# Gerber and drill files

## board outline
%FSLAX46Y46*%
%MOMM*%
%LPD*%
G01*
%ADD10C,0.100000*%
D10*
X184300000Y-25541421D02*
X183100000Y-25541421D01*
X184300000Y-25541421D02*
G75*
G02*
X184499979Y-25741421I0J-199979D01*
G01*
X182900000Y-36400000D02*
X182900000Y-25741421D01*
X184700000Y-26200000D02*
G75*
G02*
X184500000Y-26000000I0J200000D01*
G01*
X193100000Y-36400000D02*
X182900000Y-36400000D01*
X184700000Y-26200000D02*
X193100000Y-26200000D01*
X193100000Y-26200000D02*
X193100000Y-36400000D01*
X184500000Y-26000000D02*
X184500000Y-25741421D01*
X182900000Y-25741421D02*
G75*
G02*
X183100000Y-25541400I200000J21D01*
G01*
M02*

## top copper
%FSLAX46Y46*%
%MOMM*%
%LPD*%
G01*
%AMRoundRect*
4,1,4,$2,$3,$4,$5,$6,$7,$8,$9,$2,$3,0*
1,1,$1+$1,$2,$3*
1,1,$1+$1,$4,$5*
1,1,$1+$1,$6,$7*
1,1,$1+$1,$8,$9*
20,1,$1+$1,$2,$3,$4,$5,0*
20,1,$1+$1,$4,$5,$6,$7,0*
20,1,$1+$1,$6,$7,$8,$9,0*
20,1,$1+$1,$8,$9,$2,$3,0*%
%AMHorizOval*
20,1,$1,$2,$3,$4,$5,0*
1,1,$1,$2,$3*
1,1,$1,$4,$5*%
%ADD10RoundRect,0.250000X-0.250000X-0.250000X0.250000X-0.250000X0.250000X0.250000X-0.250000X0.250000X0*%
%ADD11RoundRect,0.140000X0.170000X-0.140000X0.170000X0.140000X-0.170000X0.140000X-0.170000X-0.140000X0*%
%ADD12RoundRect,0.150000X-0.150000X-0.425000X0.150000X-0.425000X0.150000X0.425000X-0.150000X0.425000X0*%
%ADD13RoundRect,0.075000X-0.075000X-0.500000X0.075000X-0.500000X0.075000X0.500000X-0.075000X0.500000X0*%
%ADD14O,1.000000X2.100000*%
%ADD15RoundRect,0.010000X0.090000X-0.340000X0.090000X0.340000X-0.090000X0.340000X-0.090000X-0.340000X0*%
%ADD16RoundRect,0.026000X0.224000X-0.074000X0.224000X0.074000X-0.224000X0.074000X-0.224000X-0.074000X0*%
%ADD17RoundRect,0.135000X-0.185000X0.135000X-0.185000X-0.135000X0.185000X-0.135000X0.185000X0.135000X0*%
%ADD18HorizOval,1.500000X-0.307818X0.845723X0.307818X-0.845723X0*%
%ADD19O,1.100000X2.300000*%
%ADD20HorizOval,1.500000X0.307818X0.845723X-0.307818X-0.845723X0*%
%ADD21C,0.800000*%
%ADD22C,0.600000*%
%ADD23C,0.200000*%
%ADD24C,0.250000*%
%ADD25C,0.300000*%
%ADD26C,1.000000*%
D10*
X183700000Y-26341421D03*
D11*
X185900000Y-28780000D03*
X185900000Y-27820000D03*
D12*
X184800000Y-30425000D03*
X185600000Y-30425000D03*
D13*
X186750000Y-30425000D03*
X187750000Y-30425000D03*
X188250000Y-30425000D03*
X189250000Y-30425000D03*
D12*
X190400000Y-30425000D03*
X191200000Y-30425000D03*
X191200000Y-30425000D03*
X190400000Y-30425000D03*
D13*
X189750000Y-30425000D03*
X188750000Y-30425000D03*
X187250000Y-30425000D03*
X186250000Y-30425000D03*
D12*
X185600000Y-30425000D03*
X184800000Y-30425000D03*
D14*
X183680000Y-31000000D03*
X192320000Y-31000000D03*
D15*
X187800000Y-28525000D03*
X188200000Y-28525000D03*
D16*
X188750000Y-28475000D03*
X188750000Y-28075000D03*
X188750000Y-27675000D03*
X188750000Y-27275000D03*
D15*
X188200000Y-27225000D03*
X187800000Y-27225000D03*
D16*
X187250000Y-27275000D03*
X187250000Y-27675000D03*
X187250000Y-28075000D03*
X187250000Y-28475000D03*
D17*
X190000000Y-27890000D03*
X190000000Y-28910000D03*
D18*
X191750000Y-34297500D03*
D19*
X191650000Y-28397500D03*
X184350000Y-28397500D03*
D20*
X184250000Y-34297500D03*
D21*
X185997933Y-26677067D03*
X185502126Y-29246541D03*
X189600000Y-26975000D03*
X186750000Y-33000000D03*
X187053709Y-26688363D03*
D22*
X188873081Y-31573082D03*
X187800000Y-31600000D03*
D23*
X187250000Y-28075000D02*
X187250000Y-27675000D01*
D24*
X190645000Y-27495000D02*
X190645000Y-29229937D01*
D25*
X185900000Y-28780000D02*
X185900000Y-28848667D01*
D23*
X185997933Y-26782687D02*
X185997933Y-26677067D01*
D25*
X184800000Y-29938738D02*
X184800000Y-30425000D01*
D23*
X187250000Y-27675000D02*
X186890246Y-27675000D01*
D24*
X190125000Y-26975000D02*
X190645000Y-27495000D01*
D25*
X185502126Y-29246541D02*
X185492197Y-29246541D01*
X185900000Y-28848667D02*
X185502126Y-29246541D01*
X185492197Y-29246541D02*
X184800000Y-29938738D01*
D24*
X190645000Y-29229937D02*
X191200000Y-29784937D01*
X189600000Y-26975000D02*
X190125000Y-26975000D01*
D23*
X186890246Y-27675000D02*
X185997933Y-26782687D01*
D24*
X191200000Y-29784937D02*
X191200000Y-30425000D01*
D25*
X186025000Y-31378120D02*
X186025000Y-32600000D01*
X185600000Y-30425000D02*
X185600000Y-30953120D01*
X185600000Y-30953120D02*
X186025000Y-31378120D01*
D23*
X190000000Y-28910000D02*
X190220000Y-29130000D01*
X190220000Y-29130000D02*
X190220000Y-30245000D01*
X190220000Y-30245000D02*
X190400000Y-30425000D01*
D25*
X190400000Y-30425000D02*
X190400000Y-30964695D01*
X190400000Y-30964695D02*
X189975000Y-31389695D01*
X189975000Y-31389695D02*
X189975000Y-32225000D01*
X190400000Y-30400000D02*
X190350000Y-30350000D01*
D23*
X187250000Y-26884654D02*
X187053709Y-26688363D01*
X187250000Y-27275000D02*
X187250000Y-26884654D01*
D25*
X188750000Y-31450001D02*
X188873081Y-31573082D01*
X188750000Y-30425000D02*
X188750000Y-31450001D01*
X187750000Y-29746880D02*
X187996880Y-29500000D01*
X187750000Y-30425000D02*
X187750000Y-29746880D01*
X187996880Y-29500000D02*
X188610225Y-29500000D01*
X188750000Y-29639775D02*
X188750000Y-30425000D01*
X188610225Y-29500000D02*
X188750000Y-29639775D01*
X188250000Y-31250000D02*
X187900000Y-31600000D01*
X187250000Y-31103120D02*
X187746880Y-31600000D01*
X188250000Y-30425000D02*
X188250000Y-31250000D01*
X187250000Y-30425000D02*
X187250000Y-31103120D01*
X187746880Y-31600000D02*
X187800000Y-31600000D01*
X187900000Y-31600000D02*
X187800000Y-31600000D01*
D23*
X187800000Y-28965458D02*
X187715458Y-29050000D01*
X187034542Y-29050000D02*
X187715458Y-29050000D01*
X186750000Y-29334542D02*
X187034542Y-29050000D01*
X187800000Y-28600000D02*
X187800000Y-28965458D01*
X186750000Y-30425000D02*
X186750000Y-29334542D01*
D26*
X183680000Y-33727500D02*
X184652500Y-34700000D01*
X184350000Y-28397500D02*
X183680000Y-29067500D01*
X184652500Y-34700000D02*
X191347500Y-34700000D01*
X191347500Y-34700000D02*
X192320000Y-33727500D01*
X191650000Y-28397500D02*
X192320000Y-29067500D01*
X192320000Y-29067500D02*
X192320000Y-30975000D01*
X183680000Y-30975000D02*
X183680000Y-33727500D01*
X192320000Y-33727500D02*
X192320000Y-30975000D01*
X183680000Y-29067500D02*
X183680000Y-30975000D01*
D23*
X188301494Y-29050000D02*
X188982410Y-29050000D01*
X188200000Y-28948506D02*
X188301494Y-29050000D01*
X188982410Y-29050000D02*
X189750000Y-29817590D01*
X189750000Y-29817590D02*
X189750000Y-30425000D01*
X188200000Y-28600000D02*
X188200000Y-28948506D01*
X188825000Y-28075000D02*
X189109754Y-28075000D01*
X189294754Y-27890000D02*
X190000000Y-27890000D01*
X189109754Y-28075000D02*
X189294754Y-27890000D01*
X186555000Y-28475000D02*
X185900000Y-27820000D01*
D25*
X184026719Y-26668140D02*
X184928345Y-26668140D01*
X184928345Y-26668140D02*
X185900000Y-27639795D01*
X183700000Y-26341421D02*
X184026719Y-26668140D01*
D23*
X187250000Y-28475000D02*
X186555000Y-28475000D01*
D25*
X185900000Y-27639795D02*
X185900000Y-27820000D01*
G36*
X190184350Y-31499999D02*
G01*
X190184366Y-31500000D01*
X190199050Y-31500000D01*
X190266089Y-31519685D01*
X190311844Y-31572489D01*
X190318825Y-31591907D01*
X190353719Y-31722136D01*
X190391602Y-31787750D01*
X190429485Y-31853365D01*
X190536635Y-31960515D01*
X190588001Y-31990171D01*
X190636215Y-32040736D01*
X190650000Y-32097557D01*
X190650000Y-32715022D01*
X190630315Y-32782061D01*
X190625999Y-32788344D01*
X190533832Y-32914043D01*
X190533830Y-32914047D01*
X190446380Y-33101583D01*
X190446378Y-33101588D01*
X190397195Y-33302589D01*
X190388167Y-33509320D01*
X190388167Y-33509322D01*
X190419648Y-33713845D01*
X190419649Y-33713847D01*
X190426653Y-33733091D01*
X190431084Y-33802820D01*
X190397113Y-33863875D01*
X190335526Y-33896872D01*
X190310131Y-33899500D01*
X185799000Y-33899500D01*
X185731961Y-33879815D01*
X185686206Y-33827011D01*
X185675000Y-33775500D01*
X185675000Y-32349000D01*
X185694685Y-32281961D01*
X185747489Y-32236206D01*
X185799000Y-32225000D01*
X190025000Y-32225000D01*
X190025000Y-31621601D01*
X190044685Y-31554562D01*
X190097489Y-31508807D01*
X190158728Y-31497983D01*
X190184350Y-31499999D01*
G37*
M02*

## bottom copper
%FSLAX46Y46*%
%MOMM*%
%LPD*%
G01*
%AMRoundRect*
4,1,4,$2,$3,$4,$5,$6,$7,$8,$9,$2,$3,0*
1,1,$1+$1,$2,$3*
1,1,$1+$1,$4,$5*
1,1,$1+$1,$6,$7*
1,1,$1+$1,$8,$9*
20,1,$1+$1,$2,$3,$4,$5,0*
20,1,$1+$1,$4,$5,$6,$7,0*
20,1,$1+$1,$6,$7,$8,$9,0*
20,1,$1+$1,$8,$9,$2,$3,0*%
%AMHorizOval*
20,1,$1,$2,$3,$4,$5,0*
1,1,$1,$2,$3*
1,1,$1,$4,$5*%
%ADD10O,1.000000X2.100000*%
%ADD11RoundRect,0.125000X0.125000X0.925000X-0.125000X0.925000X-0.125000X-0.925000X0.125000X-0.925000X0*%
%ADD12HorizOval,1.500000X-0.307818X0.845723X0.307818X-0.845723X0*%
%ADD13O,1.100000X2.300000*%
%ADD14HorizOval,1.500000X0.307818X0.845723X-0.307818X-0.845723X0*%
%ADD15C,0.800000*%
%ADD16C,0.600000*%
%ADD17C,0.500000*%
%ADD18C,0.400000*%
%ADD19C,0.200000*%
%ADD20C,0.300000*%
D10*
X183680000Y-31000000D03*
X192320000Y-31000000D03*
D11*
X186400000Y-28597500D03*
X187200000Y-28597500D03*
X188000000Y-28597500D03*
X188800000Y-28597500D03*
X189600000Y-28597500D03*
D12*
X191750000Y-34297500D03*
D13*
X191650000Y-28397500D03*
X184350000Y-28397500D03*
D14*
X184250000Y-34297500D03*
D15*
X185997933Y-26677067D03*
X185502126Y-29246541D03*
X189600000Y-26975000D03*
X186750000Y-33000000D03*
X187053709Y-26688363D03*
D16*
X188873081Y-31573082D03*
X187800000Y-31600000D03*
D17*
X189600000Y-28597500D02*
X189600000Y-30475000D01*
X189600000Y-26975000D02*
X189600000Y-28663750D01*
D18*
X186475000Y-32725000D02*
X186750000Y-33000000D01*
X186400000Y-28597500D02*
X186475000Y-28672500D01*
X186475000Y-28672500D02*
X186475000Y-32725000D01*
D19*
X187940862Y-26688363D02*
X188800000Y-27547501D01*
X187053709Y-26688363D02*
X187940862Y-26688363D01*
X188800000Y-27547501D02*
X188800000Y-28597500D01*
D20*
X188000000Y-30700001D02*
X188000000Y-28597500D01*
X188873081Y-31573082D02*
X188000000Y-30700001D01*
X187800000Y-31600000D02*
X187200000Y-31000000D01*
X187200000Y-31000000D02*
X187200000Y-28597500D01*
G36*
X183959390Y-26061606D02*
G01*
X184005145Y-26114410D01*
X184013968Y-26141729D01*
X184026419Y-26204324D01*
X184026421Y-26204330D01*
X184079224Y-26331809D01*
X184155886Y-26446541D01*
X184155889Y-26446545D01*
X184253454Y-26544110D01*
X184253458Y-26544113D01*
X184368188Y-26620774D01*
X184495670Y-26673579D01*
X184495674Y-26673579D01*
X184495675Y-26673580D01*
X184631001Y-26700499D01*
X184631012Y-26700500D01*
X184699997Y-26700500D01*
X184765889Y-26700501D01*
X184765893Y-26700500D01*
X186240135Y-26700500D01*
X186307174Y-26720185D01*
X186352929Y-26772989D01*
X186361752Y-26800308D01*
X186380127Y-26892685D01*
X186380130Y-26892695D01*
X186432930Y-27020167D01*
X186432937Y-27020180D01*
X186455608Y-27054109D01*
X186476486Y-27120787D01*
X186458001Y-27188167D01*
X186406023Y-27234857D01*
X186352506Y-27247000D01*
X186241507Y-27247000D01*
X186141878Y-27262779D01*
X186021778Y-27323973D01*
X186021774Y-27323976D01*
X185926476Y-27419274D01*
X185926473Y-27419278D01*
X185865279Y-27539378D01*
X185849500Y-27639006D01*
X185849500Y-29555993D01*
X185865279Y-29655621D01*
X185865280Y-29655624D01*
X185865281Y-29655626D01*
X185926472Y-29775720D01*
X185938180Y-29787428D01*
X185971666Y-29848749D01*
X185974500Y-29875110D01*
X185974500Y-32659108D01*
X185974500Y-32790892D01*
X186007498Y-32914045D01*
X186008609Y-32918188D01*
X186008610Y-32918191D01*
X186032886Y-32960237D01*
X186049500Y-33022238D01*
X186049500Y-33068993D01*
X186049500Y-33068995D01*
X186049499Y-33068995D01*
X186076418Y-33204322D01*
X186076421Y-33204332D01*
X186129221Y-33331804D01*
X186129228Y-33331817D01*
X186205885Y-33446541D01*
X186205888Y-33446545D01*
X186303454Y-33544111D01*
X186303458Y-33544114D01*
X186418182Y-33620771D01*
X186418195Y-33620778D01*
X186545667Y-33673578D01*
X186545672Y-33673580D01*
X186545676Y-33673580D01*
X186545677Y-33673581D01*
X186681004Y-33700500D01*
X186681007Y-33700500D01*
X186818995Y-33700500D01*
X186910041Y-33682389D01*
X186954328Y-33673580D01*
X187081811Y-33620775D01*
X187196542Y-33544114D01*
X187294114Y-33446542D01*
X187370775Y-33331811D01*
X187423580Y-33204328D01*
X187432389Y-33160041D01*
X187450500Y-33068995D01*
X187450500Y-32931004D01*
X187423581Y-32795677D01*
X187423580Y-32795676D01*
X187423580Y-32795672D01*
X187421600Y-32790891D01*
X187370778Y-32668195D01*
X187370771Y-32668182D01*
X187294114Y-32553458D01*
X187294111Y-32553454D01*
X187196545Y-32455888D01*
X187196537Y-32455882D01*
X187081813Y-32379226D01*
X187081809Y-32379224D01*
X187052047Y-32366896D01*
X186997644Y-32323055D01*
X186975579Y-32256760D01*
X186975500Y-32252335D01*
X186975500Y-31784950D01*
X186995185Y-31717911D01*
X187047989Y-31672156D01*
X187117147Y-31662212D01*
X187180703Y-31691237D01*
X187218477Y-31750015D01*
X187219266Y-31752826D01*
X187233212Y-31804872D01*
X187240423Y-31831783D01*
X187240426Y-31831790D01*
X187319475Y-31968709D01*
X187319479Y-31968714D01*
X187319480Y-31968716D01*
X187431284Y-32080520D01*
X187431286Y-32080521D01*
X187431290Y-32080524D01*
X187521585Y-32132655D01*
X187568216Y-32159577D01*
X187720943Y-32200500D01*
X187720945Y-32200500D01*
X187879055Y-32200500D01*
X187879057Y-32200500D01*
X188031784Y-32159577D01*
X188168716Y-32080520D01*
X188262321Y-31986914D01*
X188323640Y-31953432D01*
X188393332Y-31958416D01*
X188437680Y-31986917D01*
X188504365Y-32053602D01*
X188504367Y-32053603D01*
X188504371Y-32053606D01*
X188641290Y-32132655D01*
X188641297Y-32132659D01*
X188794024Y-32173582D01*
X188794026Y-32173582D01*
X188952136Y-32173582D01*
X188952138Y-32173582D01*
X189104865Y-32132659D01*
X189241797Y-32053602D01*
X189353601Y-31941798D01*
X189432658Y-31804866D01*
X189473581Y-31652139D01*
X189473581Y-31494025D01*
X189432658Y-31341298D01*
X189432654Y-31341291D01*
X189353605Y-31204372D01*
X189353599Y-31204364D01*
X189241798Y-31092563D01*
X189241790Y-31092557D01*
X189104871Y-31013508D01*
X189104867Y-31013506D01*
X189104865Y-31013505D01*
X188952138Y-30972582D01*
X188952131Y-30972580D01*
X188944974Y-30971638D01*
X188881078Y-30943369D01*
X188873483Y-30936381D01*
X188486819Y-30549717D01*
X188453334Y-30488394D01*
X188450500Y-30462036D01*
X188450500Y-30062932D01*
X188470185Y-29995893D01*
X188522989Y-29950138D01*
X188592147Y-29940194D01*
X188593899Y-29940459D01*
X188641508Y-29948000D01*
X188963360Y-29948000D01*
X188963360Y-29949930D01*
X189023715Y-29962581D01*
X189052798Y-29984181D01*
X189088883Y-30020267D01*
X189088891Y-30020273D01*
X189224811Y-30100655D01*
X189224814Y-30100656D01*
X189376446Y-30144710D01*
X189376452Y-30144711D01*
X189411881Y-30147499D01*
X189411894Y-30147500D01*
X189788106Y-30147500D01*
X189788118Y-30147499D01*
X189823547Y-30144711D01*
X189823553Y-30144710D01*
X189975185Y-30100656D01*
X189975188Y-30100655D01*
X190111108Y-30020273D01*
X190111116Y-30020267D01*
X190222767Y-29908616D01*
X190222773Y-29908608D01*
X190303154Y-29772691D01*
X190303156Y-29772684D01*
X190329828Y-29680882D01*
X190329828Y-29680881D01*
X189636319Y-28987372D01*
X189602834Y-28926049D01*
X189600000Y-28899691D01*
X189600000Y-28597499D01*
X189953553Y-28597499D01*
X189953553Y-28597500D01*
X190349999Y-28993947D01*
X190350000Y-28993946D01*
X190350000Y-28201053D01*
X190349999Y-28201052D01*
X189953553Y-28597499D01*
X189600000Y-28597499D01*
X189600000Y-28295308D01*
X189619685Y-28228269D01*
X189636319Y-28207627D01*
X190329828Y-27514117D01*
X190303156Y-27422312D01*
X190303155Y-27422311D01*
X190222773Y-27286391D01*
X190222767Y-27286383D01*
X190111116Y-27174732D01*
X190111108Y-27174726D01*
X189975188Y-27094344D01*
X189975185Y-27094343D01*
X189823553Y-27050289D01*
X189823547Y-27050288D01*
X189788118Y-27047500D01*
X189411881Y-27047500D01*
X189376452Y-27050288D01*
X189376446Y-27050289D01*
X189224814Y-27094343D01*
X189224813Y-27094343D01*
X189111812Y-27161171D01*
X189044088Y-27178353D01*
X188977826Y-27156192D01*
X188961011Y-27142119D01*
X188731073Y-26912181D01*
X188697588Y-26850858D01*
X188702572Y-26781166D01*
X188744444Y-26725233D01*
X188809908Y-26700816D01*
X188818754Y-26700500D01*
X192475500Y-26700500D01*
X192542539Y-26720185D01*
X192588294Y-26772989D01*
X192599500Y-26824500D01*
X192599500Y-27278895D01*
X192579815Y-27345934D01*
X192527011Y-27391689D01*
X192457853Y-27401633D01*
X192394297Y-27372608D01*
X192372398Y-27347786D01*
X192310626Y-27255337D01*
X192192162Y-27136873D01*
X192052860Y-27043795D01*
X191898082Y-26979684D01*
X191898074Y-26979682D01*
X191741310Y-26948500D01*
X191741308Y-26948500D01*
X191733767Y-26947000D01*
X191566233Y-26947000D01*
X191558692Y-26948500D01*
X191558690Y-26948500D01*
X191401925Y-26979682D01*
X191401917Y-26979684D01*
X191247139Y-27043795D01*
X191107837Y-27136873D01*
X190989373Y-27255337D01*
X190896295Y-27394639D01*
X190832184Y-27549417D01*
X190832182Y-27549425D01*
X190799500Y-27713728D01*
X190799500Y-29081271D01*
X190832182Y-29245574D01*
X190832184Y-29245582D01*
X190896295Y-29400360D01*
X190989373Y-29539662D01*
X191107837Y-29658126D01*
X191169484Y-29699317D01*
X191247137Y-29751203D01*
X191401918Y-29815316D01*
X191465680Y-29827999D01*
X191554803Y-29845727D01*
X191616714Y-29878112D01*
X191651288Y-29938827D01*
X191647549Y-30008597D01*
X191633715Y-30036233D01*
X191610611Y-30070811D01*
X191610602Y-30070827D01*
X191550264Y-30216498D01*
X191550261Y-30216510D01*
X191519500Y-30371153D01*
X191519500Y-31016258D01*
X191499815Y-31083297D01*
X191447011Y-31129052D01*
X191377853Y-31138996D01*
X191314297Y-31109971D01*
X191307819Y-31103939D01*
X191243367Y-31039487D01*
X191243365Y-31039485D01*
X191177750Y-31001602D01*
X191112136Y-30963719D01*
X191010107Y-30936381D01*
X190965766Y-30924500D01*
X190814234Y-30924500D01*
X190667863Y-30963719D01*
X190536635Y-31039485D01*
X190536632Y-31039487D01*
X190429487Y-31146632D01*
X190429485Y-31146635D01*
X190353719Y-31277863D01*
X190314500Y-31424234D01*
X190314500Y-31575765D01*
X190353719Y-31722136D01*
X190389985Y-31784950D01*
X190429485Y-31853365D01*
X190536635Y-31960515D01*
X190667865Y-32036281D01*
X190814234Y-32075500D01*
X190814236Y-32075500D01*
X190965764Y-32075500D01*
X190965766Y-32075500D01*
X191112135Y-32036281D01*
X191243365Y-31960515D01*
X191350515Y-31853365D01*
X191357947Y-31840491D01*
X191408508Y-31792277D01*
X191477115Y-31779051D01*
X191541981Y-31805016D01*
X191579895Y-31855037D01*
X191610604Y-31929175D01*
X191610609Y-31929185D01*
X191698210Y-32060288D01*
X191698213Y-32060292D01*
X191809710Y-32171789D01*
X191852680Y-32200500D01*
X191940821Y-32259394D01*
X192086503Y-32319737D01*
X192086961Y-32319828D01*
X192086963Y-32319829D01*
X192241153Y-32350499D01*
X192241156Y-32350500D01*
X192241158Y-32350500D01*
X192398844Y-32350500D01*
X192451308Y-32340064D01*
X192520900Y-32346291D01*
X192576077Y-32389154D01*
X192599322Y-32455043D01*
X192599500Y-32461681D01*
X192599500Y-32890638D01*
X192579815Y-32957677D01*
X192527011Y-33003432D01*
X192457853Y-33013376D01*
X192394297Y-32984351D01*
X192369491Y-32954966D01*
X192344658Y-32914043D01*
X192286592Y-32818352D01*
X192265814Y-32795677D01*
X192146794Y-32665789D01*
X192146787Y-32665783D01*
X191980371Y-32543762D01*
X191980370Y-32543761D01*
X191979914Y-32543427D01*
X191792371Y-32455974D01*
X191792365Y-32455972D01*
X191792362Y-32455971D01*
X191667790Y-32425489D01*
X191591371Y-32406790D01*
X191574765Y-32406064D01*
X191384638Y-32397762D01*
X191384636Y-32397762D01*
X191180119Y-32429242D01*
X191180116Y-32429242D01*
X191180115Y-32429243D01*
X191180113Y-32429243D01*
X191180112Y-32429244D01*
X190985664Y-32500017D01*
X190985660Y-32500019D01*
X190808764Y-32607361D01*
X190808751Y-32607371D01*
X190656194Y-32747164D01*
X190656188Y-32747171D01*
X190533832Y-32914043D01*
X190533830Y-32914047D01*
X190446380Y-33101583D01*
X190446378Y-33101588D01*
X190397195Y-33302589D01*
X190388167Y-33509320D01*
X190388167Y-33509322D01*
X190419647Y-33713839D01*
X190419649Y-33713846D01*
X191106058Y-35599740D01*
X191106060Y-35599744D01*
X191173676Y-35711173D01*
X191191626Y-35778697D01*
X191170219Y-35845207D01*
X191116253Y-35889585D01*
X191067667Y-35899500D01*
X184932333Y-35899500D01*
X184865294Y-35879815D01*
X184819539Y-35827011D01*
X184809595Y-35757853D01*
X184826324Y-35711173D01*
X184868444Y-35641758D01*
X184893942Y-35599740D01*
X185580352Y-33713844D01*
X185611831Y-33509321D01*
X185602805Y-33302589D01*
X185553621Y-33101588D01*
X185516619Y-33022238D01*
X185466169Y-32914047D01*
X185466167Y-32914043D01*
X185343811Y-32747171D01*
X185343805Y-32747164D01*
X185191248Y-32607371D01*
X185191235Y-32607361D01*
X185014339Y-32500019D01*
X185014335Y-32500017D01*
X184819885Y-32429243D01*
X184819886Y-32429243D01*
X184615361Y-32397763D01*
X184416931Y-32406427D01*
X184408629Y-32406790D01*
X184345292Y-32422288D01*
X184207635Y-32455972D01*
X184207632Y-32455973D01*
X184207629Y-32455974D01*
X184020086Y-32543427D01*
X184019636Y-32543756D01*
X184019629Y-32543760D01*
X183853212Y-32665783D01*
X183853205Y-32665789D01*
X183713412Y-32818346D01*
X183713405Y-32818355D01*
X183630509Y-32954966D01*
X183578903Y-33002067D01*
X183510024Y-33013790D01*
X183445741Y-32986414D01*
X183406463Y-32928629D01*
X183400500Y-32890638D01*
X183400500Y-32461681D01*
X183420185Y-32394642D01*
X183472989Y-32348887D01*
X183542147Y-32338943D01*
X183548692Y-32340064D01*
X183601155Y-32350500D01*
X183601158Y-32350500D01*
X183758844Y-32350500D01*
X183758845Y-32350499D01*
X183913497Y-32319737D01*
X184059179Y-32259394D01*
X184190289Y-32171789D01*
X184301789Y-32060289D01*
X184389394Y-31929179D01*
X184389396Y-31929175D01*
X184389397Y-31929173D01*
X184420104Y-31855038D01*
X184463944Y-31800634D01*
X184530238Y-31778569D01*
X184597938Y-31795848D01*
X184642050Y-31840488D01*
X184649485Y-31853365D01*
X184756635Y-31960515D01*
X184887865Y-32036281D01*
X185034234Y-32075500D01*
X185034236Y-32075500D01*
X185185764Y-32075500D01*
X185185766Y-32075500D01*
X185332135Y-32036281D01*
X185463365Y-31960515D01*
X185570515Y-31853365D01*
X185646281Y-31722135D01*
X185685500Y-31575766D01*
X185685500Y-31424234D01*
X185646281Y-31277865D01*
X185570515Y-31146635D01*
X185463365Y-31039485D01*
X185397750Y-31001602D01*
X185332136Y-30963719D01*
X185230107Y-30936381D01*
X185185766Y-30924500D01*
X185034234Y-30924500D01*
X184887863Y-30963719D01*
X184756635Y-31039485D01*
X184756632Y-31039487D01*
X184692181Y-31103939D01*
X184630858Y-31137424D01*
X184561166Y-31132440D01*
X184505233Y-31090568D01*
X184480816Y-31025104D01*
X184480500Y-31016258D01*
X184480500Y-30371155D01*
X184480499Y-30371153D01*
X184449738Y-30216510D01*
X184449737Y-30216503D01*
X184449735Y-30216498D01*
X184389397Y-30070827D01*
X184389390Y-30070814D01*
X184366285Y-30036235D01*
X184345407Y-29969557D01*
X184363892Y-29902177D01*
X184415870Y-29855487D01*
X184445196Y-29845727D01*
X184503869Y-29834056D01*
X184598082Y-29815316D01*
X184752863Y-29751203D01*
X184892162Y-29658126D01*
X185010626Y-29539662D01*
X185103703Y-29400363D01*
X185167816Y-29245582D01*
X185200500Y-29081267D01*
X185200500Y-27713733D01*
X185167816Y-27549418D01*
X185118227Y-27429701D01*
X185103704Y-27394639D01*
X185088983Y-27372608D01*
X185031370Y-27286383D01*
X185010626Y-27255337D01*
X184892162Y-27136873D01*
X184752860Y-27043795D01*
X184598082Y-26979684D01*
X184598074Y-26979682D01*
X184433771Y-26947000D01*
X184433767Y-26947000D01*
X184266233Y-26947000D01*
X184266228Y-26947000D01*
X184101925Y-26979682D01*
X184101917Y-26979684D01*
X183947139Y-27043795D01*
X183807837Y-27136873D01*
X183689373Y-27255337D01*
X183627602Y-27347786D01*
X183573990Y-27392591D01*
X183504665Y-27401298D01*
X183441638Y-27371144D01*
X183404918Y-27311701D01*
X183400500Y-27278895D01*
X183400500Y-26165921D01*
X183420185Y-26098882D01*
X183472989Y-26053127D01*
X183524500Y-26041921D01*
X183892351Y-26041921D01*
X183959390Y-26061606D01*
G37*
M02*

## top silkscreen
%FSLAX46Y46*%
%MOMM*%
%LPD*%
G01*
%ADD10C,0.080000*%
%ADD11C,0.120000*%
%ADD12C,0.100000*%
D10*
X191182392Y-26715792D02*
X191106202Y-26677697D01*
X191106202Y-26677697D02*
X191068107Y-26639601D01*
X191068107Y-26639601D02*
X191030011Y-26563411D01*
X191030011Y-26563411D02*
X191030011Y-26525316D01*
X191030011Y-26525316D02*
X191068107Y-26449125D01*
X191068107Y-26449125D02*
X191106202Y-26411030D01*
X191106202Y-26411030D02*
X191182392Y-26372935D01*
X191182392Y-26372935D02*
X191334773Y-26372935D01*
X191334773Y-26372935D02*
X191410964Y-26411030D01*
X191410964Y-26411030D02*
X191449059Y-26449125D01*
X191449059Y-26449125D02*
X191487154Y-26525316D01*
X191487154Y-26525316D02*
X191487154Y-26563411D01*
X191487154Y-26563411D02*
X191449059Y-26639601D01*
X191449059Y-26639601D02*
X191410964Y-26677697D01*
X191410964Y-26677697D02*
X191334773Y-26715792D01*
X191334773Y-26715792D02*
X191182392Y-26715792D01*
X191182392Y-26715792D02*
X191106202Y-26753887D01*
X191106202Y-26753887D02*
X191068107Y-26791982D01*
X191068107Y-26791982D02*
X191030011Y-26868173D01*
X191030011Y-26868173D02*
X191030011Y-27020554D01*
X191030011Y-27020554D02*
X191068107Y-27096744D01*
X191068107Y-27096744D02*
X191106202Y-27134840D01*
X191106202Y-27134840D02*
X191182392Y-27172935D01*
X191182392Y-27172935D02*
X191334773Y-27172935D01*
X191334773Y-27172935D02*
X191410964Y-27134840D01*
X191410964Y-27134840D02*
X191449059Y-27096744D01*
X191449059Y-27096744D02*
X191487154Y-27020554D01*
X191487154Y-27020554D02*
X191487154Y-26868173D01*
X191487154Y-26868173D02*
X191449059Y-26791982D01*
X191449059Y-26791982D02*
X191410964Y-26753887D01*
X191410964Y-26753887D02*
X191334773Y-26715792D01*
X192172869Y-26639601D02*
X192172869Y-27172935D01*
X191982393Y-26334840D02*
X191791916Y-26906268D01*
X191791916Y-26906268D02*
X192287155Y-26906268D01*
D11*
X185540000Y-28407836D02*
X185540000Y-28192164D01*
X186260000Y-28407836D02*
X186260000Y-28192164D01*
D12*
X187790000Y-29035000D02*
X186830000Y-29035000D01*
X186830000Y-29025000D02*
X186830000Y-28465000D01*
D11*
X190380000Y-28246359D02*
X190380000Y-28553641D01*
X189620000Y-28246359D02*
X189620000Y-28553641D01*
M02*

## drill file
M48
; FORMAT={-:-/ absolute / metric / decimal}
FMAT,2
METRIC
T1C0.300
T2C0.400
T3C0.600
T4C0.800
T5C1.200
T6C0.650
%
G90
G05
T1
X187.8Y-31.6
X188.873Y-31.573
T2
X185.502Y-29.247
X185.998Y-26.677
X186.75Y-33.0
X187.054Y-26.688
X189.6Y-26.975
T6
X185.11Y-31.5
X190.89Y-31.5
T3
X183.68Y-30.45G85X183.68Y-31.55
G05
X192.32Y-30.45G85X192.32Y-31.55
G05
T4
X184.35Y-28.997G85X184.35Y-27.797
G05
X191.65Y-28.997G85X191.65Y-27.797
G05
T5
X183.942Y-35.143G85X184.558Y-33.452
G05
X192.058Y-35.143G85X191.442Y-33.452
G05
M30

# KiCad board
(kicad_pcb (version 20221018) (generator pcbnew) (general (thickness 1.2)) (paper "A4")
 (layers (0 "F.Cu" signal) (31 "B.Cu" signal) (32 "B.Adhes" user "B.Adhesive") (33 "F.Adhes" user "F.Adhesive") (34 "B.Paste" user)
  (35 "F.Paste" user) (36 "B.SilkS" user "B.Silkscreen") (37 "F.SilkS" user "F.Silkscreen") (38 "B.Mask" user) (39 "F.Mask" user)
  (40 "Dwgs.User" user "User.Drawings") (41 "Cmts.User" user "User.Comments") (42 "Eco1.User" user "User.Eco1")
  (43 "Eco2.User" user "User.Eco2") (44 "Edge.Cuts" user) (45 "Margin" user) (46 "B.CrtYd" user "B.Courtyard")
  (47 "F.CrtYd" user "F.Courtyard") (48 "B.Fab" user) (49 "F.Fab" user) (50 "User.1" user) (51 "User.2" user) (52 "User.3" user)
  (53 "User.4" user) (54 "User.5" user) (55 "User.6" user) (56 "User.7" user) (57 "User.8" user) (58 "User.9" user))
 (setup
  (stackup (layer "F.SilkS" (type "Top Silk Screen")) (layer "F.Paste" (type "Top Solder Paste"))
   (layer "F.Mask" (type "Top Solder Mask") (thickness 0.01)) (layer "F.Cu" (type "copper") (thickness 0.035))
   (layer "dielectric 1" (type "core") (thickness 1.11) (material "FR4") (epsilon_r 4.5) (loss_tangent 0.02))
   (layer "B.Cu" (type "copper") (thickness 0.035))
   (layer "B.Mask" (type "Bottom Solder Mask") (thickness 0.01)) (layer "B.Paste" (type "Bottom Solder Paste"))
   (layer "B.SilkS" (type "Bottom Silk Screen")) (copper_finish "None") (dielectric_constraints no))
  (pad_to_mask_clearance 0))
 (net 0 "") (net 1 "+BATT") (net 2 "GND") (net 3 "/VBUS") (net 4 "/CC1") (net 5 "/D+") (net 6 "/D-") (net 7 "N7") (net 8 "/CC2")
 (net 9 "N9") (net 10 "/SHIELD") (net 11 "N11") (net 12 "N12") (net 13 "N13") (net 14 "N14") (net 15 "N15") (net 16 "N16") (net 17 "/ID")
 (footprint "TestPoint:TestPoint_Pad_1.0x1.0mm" (layer "F.Cu") (at 183.7 26.341421)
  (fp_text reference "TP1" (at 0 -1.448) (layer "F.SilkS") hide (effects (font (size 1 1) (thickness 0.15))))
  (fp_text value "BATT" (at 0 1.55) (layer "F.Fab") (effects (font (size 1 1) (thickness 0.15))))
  (pad "1" smd roundrect (at 0 0) (size 1 1) (layers "F.Cu" "F.Mask") (roundrect_rratio 0.25) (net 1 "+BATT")))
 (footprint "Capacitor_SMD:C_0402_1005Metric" (layer "F.Cu") (at 185.9 28.3 90)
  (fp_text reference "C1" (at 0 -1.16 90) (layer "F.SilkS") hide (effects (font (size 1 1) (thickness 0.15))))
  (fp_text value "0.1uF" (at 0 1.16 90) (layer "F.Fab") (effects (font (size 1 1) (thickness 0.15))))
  (fp_line (start -0.107836 -0.36) (end 0.107836 -0.36) (stroke (width 0.12) (type solid)) (layer "F.SilkS"))
  (fp_line (start -0.107836 0.36) (end 0.107836 0.36) (stroke (width 0.12) (type solid)) (layer "F.SilkS"))
  (pad "1" smd roundrect (at -0.48 0 90) (size 0.56 0.62) (layers "F.Cu" "F.Paste" "F.Mask") (roundrect_rratio 0.25) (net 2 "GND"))
  (pad "2" smd roundrect (at 0.48 0 90) (size 0.56 0.62) (layers "F.Cu" "F.Paste" "F.Mask") (roundrect_rratio 0.25) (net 1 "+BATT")))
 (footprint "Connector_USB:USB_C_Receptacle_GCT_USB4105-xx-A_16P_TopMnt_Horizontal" (layer "F.Cu") (at 188 34.105)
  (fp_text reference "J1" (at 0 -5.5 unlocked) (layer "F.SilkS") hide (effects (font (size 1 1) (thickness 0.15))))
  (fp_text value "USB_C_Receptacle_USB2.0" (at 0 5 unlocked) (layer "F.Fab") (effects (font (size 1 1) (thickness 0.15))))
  (pad "" np_thru_hole circle (at -2.89 -2.605) (size 0.65 0.65) (drill 0.65) (layers "F&B.Cu" "*.Mask"))
  (pad "" np_thru_hole circle (at 2.89 -2.605) (size 0.65 0.65) (drill 0.65) (layers "F&B.Cu" "*.Mask"))
  (pad "A1" smd roundrect (at -3.2 -3.68) (size 0.6 1.15) (layers "F.Cu" "F.Paste" "F.Mask") (roundrect_rratio 0.25) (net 2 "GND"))
  (pad "A4" smd roundrect (at -2.4 -3.68) (size 0.6 1.15) (layers "F.Cu" "F.Paste" "F.Mask") (roundrect_rratio 0.25) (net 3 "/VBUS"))
  (pad "A5" smd roundrect (at -1.25 -3.68) (size 0.3 1.15) (layers "F.Cu" "F.Paste" "F.Mask") (roundrect_rratio 0.25) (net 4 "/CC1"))
  (pad "A6" smd roundrect (at -0.25 -3.68) (size 0.3 1.15) (layers "F.Cu" "F.Paste" "F.Mask") (roundrect_rratio 0.25) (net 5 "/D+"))
  (pad "A7" smd roundrect (at 0.25 -3.68) (size 0.3 1.15) (layers "F.Cu" "F.Paste" "F.Mask") (roundrect_rratio 0.25) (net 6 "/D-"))
  (pad "A8" smd roundrect (at 1.25 -3.68) (size 0.3 1.15) (layers "F.Cu" "F.Paste" "F.Mask") (roundrect_rratio 0.25) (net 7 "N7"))
  (pad "A9" smd roundrect (at 2.4 -3.68) (size 0.6 1.15) (layers "F.Cu" "F.Paste" "F.Mask") (roundrect_rratio 0.25) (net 3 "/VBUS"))
  (pad "A12" smd roundrect (at 3.2 -3.68) (size 0.6 1.15) (layers "F.Cu" "F.Paste" "F.Mask") (roundrect_rratio 0.25) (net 2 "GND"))
  (pad "B1" smd roundrect (at 3.2 -3.68) (size 0.6 1.15) (layers "F.Cu" "F.Paste" "F.Mask") (roundrect_rratio 0.25) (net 2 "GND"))
  (pad "B4" smd roundrect (at 2.4 -3.68) (size 0.6 1.15) (layers "F.Cu" "F.Paste" "F.Mask") (roundrect_rratio 0.25) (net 3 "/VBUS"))
  (pad "B5" smd roundrect (at 1.75 -3.68) (size 0.3 1.15) (layers "F.Cu" "F.Paste" "F.Mask") (roundrect_rratio 0.25) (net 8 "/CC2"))
  (pad "B6" smd roundrect (at 0.75 -3.68) (size 0.3 1.15) (layers "F.Cu" "F.Paste" "F.Mask") (roundrect_rratio 0.25) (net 5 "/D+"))
  (pad "B7" smd roundrect (at -0.75 -3.68) (size 0.3 1.15) (layers "F.Cu" "F.Paste" "F.Mask") (roundrect_rratio 0.25) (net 6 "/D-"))
  (pad "B8" smd roundrect (at -1.75 -3.68) (size 0.3 1.15) (layers "F.Cu" "F.Paste" "F.Mask") (roundrect_rratio 0.25) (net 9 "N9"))
  (pad "B9" smd roundrect (at -2.4 -3.68) (size 0.6 1.15) (layers "F.Cu" "F.Paste" "F.Mask") (roundrect_rratio 0.25) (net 3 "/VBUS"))
  (pad "B12" smd roundrect (at -3.2 -3.68) (size 0.6 1.15) (layers "F.Cu" "F.Paste" "F.Mask") (roundrect_rratio 0.25) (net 2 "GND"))
  (pad "S1" thru_hole oval (at -4.32 -3.105) (size 1 2.1) (drill oval 0.6 1.7) (layers "*.Cu" "*.Mask" "F.Paste") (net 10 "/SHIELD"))
  (pad "S1" thru_hole oval (at 4.32 -3.105) (size 1 2.1) (drill oval 0.6 1.7) (layers "*.Cu" "*.Mask" "F.Paste") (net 10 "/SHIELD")))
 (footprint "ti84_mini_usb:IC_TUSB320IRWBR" (layer "F.Cu") (at 188 27.875 90)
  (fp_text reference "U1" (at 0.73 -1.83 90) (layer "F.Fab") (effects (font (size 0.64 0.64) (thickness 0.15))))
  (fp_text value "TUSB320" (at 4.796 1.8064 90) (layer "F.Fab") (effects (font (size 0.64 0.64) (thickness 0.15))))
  (fp_line (start -1.16 -0.21) (end -1.16 -1.17) (stroke (width 0.1) (type default)) (layer "F.SilkS"))
  (fp_line (start -1.15 -1.17) (end -0.59 -1.17) (stroke (width 0.1) (type default)) (layer "F.SilkS"))
  (pad "1" smd roundrect (at -0.65 -0.2 90) (size 0.7 0.2) (layers "F.Cu") (roundrect_rratio 0.05) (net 4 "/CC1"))
  (pad "2" smd roundrect (at -0.65 0.2 90) (size 0.7 0.2) (layers "F.Cu") (roundrect_rratio 0.05) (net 8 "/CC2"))
  (pad "3" smd roundrect (at -0.6 0.75 90) (size 0.2 0.5) (layers "F.Cu" "F.Paste") (roundrect_rratio 0.13) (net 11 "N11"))
  (pad "4" smd roundrect (at -0.2 0.75 90) (size 0.2 0.5) (layers "F.Cu" "F.Paste") (roundrect_rratio 0.13) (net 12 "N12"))
  (pad "5" smd roundrect (at 0.2 0.75 90) (size 0.2 0.5) (layers "F.Cu" "F.Paste") (roundrect_rratio 0.13) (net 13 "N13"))
  (pad "6" smd roundrect (at 0.6 0.75 90) (size 0.2 0.5) (layers "F.Cu" "F.Paste") (roundrect_rratio 0.13) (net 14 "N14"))
  (pad "7" smd roundrect (at 0.65 0.2 90) (size 0.7 0.2) (layers "F.Cu") (roundrect_rratio 0.05) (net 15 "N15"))
  (pad "8" smd roundrect (at 0.65 -0.2 90) (size 0.7 0.2) (layers "F.Cu") (roundrect_rratio 0.05) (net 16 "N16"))
  (pad "9" smd roundrect (at 0.6 -0.75 90) (size 0.2 0.5) (layers "F.Cu" "F.Paste") (roundrect_rratio 0.13) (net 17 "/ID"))
  (pad "10" smd roundrect (at 0.2 -0.75 90) (size 0.2 0.5) (layers "F.Cu" "F.Paste") (roundrect_rratio 0.13) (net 2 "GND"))
  (pad "11" smd roundrect (at -0.2 -0.75 90) (size 0.2 0.5) (layers "F.Cu" "F.Paste") (roundrect_rratio 0.13) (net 2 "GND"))
  (pad "12" smd roundrect (at -0.6 -0.75 90) (size 0.2 0.5) (layers "F.Cu" "F.Paste") (roundrect_rratio 0.13) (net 1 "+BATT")))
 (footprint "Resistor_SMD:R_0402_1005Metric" (layer "F.Cu") (at 190 28.4 -90)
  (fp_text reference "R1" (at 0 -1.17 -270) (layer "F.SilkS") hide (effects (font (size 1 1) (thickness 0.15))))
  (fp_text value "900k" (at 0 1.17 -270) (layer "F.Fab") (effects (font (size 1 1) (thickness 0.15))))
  (fp_line (start -0.153641 -0.38) (end 0.153641 -0.38) (stroke (width 0.12) (type solid)) (layer "F.SilkS"))
  (fp_line (start -0.153641 0.38) (end 0.153641 0.38) (stroke (width 0.12) (type solid)) (layer "F.SilkS"))
  (pad "1" smd roundrect (at -0.51 0 270) (size 0.54 0.64) (layers "F.Cu" "F.Paste" "F.Mask") (roundrect_rratio 0.25) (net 12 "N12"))
  (pad "2" smd roundrect (at 0.51 0 270) (size 0.54 0.64) (layers "F.Cu" "F.Paste" "F.Mask") (roundrect_rratio 0.25) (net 3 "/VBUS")))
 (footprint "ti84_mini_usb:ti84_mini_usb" (layer "B.Cu") (at 188.25 38.1975 180)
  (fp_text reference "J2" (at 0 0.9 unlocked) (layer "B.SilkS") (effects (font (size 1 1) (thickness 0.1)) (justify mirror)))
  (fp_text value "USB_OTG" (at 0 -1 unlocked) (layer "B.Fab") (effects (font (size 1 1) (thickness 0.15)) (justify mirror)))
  (pad "1" smd roundrect (at 1.85 9.6 180) (size 0.5 2.1) (layers "B.Cu" "B.Paste" "B.Mask") (roundrect_rratio 0.25) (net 3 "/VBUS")
   (thermal_bridge_angle 45))
  (pad "2" smd roundrect (at 1.05 9.6 180) (size 0.5 2.1) (layers "B.Cu" "B.Paste" "B.Mask") (roundrect_rratio 0.25) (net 6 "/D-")
   (thermal_bridge_angle 45))
  (pad "3" smd roundrect (at 0.25 9.6 180) (size 0.5 2.1) (layers "B.Cu" "B.Paste" "B.Mask") (roundrect_rratio 0.25) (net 5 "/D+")
   (thermal_bridge_angle 45))
  (pad "4" smd roundrect (at -0.55 9.6 180) (size 0.5 2.1) (layers "B.Cu" "B.Paste" "B.Mask") (roundrect_rratio 0.25) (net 17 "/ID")
   (thermal_bridge_angle 45))
  (pad "5" smd roundrect (at -1.35 9.6 180) (size 0.5 2.1) (layers "B.Cu" "B.Paste" "B.Mask") (roundrect_rratio 0.25) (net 2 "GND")
   (thermal_bridge_angle 45))
  (pad "6" thru_hole oval (at -3.5 3.9 200) (size 1.5 3.3) (drill oval 1.2 3) (layers "*.Cu" "*.Mask") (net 10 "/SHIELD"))
  (pad "6" thru_hole oval (at -3.4 9.8 180) (size 1.1 2.3) (drill oval 0.8 2) (layers "*.Cu" "*.Mask") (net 10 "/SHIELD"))
  (pad "6" thru_hole oval (at 3.9 9.8 180) (size 1.1 2.3) (drill oval 0.8 2) (layers "*.Cu" "*.Mask") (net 10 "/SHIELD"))
  (pad "6" thru_hole oval (at 4 3.9 160) (size 1.5 3.3) (drill oval 1.2 3) (layers "*.Cu" "*.Mask") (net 10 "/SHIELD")))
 (gr_line (start 184.3 25.541421) (end 183.1 25.541421) (stroke (width 0.1) (type default)) (layer "Edge.Cuts"))
 (gr_arc (start 184.3 25.541421) (mid 184.441421 25.6) (end 184.5 25.741421) (stroke (width 0.1) (type default)) (layer "Edge.Cuts"))
 (gr_line (start 182.9 36.4) (end 182.9 25.741421) (stroke (width 0.1) (type default)) (layer "Edge.Cuts"))
 (gr_arc (start 184.7 26.2) (mid 184.558579 26.141421) (end 184.5 26) (stroke (width 0.1) (type default)) (layer "Edge.Cuts"))
 (gr_line (start 193.1 36.4) (end 182.9 36.4) (stroke (width 0.1) (type default)) (layer "Edge.Cuts"))
 (gr_line (start 184.7 26.2) (end 193.1 26.2) (stroke (width 0.1) (type default)) (layer "Edge.Cuts"))
 (gr_line (start 193.1 26.2) (end 193.1 36.4) (stroke (width 0.1) (type default)) (layer "Edge.Cuts"))
 (gr_line (start 184.5 26) (end 184.5 25.741421) (stroke (width 0.1) (type default)) (layer "Edge.Cuts"))
 (gr_arc (start 182.9 25.741421) (mid 182.958579 25.6) (end 183.1 25.541421) (stroke (width 0.1) (type default)) (layer "Edge.Cuts"))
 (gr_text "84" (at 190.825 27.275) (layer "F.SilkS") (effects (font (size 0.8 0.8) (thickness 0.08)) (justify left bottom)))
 (segment (start 187.25 28.075) (end 187.25 27.675) (width 0.2) (layer "F.Cu") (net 2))
 (segment (start 190.645 27.495) (end 190.645 29.229937) (width 0.25) (layer "F.Cu") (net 2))
 (segment (start 185.9 28.78) (end 185.9 28.848667) (width 0.3) (layer "F.Cu") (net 2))
 (segment (start 185.997933 26.782687) (end 185.997933 26.677067) (width 0.2) (layer "F.Cu") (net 2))
 (segment (start 184.8 29.938738) (end 184.8 30.425) (width 0.3) (layer "F.Cu") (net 2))
 (segment (start 187.25 27.675) (end 186.890246 27.675) (width 0.2) (layer "F.Cu") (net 2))
 (segment (start 190.125 26.975) (end 190.645 27.495) (width 0.25) (layer "F.Cu") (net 2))
 (segment (start 185.502126 29.246541) (end 185.492197 29.246541) (width 0.3) (layer "F.Cu") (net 2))
 (segment (start 185.9 28.848667) (end 185.502126 29.246541) (width 0.3) (layer "F.Cu") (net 2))
 (segment (start 185.492197 29.246541) (end 184.8 29.938738) (width 0.3) (layer "F.Cu") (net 2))
 (segment (start 190.645 29.229937) (end 191.2 29.784937) (width 0.25) (layer "F.Cu") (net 2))
 (segment (start 189.6 26.975) (end 190.125 26.975) (width 0.25) (layer "F.Cu") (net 2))
 (segment (start 186.890246 27.675) (end 185.997933 26.782687) (width 0.2) (layer "F.Cu") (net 2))
 (segment (start 191.2 29.784937) (end 191.2 30.425) (width 0.25) (layer "F.Cu") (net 2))
 (via (at 185.997933 26.677067) (size 0.8) (drill 0.4) (layers "F.Cu" "B.Cu") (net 2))
 (via (at 185.502126 29.246541) (size 0.8) (drill 0.4) (layers "F.Cu" "B.Cu") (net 2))
 (via (at 189.6 26.975) (size 0.8) (drill 0.4) (layers "F.Cu" "B.Cu") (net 2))
 (segment (start 189.6 28.5975) (end 189.6 30.475) (width 0.5) (layer "B.Cu") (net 2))
 (segment (start 189.6 26.975) (end 189.6 28.66375) (width 0.5) (layer "B.Cu") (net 2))
 (segment (start 186.025 31.37812) (end 186.025 32.6) (width 0.3) (layer "F.Cu") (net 3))
 (segment (start 185.6 30.425) (end 185.6 30.95312) (width 0.3) (layer "F.Cu") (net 3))
 (segment (start 185.6 30.95312) (end 186.025 31.37812) (width 0.3) (layer "F.Cu") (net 3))
 (segment (start 190 28.91) (end 190.22 29.13) (width 0.2) (layer "F.Cu") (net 3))
 (segment (start 190.22 29.13) (end 190.22 30.245) (width 0.2) (layer "F.Cu") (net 3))
 (segment (start 190.22 30.245) (end 190.4 30.425) (width 0.2) (layer "F.Cu") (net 3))
 (segment (start 190.4 30.425) (end 190.4 30.964695) (width 0.3) (layer "F.Cu") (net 3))
 (segment (start 190.4 30.964695) (end 189.975 31.389695) (width 0.3) (layer "F.Cu") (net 3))
 (segment (start 189.975 31.389695) (end 189.975 32.225) (width 0.3) (layer "F.Cu") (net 3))
 (segment (start 190.4 30.4) (end 190.35 30.35) (width 0.3) (layer "F.Cu") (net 3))
 (via (at 186.75 33) (size 0.8) (drill 0.4) (layers "F.Cu" "B.Cu") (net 3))
 (segment (start 186.475 32.725) (end 186.75 33) (width 0.4) (layer "B.Cu") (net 3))
 (segment (start 186.4 28.5975) (end 186.475 28.6725) (width 0.4) (layer "B.Cu") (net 3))
 (segment (start 186.475 28.6725) (end 186.475 32.725) (width 0.4) (layer "B.Cu") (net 3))
 (segment (start 187.25 26.884654) (end 187.053709 26.688363) (width 0.2) (layer "F.Cu") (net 17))
 (segment (start 187.25 27.275) (end 187.25 26.884654) (width 0.2) (layer "F.Cu") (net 17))
 (via (at 187.053709 26.688363) (size 0.8) (drill 0.4) (layers "F.Cu" "B.Cu") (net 17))
 (segment (start 187.940862 26.688363) (end 188.8 27.547501) (width 0.2) (layer "B.Cu") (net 17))
 (segment (start 187.053709 26.688363) (end 187.940862 26.688363) (width 0.2) (layer "B.Cu") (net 17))
 (segment (start 188.8 27.547501) (end 188.8 28.5975) (width 0.2) (layer "B.Cu") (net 17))
 (segment (start 188.75 31.450001) (end 188.873081 31.573082) (width 0.3) (layer "F.Cu") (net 5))
 (segment (start 188.75 30.425) (end 188.75 31.450001) (width 0.3) (layer "F.Cu") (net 5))
 (segment (start 187.75 29.74688) (end 187.99688 29.5) (width 0.3) (layer "F.Cu") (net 5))
 (segment (start 187.75 30.425) (end 187.75 29.74688) (width 0.3) (layer "F.Cu") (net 5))
 (segment (start 187.99688 29.5) (end 188.610225 29.5) (width 0.3) (layer "F.Cu") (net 5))
 (segment (start 188.75 29.639775) (end 188.75 30.425) (width 0.3) (layer "F.Cu") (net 5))
 (segment (start 188.610225 29.5) (end 188.75 29.639775) (width 0.3) (layer "F.Cu") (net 5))
 (via (at 188.873081 31.573082) (size 0.6) (drill 0.3) (layers "F.Cu" "B.Cu") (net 5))
 (segment (start 188 30.700001) (end 188 28.5975) (width 0.3) (layer "B.Cu") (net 5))
 (segment (start 188.873081 31.573082) (end 188 30.700001) (width 0.3) (layer "B.Cu") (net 5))
 (segment (start 188.25 31.25) (end 187.9 31.6) (width 0.3) (layer "F.Cu") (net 6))
 (segment (start 187.25 31.10312) (end 187.74688 31.6) (width 0.3) (layer "F.Cu") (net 6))
 (segment (start 188.25 30.425) (end 188.25 31.25) (width 0.3) (layer "F.Cu") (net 6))
 (segment (start 187.25 30.425) (end 187.25 31.10312) (width 0.3) (layer "F.Cu") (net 6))
 (segment (start 187.74688 31.6) (end 187.8 31.6) (width 0.3) (layer "F.Cu") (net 6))
 (segment (start 187.9 31.6) (end 187.8 31.6) (width 0.3) (layer "F.Cu") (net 6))
 (via (at 187.8 31.6) (size 0.6) (drill 0.3) (layers "F.Cu" "B.Cu") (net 6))
 (segment (start 187.8 31.6) (end 187.2 31) (width 0.3) (layer "B.Cu") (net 6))
 (segment (start 187.2 31) (end 187.2 28.5975) (width 0.3) (layer "B.Cu") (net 6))
 (segment (start 187.8 28.965458) (end 187.715458 29.05) (width 0.2) (layer "F.Cu") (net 4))
 (segment (start 187.034542 29.05) (end 187.715458 29.05) (width 0.2) (layer "F.Cu") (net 4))
 (segment (start 186.75 29.334542) (end 187.034542 29.05) (width 0.2) (layer "F.Cu") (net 4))
 (segment (start 187.8 28.6) (end 187.8 28.965458) (width 0.2) (layer "F.Cu") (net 4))
 (segment (start 186.75 30.425) (end 186.75 29.334542) (width 0.2) (layer "F.Cu") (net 4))
 (segment (start 183.68 33.7275) (end 184.6525 34.7) (width 1) (layer "F.Cu") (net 10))
 (segment (start 184.35 28.3975) (end 183.68 29.0675) (width 1) (layer "F.Cu") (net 10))
 (segment (start 184.6525 34.7) (end 191.3475 34.7) (width 1) (layer "F.Cu") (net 10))
 (segment (start 191.3475 34.7) (end 192.32 33.7275) (width 1) (layer "F.Cu") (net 10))
 (segment (start 191.65 28.3975) (end 192.32 29.0675) (width 1) (layer "F.Cu") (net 10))
 (segment (start 192.32 29.0675) (end 192.32 30.975) (width 1) (layer "F.Cu") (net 10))
 (segment (start 183.68 30.975) (end 183.68 33.7275) (width 1) (layer "F.Cu") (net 10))
 (segment (start 192.32 33.7275) (end 192.32 30.975) (width 1) (layer "F.Cu") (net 10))
 (segment (start 183.68 29.0675) (end 183.68 30.975) (width 1) (layer "F.Cu") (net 10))
 (segment (start 188.301494 29.05) (end 188.98241 29.05) (width 0.2) (layer "F.Cu") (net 8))
 (segment (start 188.2 28.948506) (end 188.301494 29.05) (width 0.2) (layer "F.Cu") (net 8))
 (segment (start 188.98241 29.05) (end 189.75 29.81759) (width 0.2) (layer "F.Cu") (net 8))
 (segment (start 189.75 29.81759) (end 189.75 30.425) (width 0.2) (layer "F.Cu") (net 8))
 (segment (start 188.2 28.6) (end 188.2 28.948506) (width 0.2) (layer "F.Cu") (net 8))
 (segment (start 188.825 28.075) (end 189.109754 28.075) (width 0.2) (layer "F.Cu") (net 12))
 (segment (start 189.294754 27.89) (end 190 27.89) (width 0.2) (layer "F.Cu") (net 12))
 (segment (start 189.109754 28.075) (end 189.294754 27.89) (width 0.2) (layer "F.Cu") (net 12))
 (segment (start 186.555 28.475) (end 185.9 27.82) (width 0.2) (layer "F.Cu") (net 1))
 (segment (start 184.026719 26.66814) (end 184.928345 26.66814) (width 0.3) (layer "F.Cu") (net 1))
 (segment (start 184.928345 26.66814) (end 185.9 27.639795) (width 0.3) (layer "F.Cu") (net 1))
 (segment (start 183.7 26.341421) (end 184.026719 26.66814) (width 0.3) (layer "F.Cu") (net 1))
 (segment (start 187.25 28.475) (end 186.555 28.475) (width 0.2) (layer "F.Cu") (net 1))
 (segment (start 185.9 27.639795) (end 185.9 27.82) (width 0.3) (layer "F.Cu") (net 1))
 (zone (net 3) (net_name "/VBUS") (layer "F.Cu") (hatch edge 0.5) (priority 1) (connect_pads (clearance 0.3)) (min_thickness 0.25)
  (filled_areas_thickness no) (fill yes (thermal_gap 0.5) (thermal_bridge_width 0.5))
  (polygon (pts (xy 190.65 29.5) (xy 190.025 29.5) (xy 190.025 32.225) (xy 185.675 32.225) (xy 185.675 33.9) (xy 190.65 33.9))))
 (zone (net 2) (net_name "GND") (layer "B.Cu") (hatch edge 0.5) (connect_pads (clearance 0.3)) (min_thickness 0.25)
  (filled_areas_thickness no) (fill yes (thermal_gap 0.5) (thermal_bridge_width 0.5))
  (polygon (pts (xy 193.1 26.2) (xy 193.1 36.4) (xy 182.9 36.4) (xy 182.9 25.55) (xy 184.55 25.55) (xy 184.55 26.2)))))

